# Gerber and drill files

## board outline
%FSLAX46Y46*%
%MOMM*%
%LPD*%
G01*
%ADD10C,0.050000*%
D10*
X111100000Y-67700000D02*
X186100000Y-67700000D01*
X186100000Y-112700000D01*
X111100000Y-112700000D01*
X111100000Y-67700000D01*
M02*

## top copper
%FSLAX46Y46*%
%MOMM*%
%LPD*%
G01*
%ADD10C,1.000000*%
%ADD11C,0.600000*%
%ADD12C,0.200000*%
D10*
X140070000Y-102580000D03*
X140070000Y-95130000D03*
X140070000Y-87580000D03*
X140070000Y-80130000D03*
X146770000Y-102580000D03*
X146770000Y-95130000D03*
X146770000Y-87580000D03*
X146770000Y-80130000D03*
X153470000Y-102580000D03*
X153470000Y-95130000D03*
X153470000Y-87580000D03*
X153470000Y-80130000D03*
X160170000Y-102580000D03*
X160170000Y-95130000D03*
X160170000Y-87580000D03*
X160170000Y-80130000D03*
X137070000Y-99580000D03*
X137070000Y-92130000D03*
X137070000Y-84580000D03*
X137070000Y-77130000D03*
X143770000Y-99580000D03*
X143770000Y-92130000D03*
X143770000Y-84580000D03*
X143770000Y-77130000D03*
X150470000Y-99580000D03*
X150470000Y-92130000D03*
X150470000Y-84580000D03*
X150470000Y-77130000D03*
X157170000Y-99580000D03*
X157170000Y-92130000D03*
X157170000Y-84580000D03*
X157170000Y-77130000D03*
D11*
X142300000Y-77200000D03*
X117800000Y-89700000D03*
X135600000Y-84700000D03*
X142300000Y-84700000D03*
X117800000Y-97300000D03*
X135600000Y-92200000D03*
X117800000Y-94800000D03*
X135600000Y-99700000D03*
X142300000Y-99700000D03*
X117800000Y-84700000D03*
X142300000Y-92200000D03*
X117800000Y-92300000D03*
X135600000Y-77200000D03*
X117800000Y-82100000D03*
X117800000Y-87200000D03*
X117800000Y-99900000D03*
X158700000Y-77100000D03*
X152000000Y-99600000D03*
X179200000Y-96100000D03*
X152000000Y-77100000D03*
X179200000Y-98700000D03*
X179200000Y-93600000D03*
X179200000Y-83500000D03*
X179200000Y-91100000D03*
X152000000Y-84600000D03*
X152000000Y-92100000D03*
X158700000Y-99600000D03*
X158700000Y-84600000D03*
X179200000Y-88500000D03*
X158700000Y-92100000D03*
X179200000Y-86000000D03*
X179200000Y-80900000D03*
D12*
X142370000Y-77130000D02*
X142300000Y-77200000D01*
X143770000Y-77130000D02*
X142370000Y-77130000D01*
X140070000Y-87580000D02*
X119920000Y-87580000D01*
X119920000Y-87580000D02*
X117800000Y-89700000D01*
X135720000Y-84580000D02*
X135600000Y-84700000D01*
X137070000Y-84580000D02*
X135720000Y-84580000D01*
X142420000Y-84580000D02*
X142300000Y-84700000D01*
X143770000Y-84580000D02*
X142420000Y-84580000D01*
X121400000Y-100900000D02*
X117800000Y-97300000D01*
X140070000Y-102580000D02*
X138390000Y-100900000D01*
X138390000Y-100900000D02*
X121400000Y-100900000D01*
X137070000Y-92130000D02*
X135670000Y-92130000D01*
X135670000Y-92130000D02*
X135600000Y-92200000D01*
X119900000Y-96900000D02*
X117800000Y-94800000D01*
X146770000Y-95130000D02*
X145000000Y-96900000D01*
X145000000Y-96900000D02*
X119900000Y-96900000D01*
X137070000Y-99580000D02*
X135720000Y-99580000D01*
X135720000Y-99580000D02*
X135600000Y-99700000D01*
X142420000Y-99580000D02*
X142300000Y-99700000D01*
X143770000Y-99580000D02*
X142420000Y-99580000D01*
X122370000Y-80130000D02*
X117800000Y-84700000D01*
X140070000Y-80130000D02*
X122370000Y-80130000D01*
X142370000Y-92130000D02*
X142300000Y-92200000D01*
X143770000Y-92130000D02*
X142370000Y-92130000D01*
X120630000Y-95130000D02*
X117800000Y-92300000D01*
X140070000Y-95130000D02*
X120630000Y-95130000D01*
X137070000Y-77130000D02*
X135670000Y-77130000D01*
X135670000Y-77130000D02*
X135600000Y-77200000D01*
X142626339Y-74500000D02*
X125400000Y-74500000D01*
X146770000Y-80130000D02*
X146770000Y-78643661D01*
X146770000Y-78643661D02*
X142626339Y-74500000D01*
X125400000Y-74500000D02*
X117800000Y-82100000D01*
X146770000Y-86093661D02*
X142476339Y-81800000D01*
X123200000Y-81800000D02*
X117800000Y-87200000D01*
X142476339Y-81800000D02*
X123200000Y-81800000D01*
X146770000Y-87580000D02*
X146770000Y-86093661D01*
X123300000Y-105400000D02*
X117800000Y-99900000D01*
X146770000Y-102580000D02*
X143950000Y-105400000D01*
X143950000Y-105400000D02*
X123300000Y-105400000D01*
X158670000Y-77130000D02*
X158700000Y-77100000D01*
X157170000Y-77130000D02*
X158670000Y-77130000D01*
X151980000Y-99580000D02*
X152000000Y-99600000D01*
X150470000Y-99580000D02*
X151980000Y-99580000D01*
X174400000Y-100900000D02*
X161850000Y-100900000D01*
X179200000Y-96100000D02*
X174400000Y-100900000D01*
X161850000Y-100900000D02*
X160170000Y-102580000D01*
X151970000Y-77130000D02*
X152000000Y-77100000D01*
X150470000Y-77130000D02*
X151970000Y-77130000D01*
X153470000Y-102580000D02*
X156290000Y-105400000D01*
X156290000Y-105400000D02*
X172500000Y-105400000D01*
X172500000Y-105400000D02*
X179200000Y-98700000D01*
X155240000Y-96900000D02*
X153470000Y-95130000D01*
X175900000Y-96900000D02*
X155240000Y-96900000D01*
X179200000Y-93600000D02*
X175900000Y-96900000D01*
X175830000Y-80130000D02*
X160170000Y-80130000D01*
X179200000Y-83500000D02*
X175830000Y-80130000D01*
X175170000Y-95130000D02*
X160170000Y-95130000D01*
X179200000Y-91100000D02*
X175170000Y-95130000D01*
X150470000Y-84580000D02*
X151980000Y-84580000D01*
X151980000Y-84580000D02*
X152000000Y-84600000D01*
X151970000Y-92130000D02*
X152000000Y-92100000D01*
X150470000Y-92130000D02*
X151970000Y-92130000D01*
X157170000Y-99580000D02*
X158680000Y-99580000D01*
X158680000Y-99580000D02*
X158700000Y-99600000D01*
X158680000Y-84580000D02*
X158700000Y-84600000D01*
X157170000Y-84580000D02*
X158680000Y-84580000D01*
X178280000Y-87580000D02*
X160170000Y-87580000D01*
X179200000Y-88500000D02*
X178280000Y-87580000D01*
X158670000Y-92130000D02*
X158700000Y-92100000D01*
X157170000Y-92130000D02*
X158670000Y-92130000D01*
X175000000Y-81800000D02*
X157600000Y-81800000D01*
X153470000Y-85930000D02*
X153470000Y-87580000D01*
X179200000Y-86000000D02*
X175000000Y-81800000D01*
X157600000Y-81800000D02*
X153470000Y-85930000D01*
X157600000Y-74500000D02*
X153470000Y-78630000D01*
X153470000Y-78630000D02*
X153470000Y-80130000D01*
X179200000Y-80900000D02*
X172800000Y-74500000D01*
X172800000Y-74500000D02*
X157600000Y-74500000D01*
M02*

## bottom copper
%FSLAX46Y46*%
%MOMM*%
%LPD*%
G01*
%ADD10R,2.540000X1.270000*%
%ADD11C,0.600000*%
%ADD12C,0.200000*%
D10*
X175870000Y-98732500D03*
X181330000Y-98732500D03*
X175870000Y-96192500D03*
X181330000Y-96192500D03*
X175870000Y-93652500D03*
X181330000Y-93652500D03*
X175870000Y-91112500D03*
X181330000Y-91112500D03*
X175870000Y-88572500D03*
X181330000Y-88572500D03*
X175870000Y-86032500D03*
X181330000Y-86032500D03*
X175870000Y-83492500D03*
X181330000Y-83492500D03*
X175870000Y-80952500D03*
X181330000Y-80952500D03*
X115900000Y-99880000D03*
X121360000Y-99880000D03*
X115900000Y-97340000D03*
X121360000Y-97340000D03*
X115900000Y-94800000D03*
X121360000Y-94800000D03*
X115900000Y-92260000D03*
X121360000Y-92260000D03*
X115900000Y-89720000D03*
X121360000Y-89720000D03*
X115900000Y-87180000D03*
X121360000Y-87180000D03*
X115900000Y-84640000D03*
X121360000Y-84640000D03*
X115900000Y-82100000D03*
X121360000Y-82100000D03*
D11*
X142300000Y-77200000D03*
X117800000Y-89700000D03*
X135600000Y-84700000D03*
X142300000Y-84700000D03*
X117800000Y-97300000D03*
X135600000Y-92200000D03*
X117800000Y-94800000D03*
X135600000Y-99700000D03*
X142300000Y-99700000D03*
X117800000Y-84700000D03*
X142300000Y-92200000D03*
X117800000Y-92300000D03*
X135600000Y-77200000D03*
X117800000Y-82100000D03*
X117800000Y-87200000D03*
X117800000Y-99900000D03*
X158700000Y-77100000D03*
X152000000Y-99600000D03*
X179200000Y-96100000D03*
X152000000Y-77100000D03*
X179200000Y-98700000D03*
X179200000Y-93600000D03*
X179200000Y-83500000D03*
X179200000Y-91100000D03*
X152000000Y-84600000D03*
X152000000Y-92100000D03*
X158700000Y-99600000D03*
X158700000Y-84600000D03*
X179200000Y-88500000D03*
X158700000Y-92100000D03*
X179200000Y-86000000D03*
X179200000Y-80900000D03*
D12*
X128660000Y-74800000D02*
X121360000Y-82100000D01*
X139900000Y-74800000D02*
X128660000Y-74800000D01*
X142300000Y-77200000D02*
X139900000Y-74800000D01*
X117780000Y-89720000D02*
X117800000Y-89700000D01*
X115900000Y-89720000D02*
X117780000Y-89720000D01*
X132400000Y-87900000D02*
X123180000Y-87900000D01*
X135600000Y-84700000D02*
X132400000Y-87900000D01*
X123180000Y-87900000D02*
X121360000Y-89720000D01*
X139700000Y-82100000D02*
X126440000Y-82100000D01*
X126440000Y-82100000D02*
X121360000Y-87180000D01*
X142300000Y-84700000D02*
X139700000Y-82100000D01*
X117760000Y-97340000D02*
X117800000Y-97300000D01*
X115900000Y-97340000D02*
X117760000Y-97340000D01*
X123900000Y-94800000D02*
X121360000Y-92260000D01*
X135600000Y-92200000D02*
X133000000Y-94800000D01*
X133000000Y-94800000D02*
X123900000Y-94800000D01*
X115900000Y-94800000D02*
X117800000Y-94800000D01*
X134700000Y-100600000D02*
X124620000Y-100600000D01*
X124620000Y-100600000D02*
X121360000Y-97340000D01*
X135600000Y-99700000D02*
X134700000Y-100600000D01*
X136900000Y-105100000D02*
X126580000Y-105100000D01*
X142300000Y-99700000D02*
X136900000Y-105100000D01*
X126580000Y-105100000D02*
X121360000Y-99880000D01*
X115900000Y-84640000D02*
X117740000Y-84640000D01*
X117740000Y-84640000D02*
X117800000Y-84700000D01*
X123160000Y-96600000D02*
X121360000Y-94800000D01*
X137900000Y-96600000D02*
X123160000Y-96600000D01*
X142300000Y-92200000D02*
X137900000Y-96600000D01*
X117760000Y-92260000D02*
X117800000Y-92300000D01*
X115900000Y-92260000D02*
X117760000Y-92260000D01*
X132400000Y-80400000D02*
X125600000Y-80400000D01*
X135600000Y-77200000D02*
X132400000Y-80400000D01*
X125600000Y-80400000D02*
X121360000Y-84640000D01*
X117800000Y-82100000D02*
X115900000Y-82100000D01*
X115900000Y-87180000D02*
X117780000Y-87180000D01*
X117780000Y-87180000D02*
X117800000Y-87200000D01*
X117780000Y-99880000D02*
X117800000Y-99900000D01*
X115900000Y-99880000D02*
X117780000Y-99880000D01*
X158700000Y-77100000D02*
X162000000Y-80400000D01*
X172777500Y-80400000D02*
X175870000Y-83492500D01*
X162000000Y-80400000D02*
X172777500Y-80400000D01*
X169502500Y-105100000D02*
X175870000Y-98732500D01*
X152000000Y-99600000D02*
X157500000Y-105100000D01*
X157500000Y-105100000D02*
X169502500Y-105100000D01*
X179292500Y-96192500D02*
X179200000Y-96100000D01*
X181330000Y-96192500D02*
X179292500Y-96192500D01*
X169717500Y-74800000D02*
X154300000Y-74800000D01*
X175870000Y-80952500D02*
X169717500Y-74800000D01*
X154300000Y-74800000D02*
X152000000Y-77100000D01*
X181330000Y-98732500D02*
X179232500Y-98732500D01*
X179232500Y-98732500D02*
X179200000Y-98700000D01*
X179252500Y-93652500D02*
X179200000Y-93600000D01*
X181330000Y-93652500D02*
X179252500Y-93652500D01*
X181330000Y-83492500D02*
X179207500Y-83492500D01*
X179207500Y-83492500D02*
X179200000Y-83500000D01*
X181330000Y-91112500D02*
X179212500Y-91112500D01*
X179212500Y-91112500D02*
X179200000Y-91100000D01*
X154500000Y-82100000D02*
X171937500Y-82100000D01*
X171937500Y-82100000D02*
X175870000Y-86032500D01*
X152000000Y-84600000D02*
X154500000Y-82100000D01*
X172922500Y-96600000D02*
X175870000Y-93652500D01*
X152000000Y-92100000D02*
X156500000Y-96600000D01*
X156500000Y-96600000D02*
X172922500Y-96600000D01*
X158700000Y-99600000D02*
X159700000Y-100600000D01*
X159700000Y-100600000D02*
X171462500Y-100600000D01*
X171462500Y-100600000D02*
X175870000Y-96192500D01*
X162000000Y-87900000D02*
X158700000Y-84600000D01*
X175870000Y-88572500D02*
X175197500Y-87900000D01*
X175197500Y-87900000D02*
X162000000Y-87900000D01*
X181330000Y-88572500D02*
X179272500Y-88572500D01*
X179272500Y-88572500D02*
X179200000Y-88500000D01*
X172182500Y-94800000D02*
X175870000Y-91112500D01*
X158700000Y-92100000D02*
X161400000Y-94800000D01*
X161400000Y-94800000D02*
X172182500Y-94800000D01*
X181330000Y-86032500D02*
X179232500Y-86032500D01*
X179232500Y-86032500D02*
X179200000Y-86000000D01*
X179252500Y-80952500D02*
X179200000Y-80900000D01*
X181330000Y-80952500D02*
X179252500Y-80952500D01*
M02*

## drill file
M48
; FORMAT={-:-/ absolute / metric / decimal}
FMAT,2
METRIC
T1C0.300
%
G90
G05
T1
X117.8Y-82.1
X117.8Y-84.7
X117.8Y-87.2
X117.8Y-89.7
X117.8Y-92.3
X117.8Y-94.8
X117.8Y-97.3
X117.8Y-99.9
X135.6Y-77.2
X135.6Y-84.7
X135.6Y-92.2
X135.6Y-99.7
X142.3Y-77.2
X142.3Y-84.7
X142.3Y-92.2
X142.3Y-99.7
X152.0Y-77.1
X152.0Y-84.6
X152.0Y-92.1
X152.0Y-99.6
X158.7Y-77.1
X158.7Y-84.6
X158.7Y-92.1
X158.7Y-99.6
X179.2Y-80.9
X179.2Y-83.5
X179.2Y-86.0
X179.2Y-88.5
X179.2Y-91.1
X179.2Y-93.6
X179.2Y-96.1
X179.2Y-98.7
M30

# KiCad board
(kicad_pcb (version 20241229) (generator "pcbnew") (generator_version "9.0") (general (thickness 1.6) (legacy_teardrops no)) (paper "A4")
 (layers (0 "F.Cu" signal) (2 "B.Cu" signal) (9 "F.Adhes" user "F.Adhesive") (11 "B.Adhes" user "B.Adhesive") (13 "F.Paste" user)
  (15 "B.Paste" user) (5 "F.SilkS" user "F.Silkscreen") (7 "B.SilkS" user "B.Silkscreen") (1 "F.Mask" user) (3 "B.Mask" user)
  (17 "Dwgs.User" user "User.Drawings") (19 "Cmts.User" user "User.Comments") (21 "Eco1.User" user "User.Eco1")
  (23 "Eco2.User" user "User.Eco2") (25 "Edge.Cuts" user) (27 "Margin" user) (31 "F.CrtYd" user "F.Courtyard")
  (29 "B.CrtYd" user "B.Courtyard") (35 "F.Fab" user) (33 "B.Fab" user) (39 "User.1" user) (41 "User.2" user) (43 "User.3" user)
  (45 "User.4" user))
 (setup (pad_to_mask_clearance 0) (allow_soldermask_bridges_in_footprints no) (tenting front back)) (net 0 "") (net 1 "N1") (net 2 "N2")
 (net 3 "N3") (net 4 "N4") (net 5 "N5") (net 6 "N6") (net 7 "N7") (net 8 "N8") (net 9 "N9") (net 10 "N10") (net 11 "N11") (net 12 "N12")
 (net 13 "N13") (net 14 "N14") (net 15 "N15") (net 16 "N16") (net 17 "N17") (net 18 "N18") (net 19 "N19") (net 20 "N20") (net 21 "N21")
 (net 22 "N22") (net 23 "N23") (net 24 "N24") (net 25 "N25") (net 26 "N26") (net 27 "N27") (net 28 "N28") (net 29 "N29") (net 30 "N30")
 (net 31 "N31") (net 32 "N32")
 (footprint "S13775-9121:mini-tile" (layer "F.Cu") (at 148.62 90.13)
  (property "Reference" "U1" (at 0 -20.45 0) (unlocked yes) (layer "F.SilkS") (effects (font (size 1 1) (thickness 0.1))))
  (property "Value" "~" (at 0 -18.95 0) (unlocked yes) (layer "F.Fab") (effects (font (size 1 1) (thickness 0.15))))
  (pad "AA1" smd circle (at -8.55 12.45) (size 1 1) (layers "F.Cu" "F.Mask" "F.Paste") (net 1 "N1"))
  (pad "AA2" smd circle (at -8.55 5) (size 1 1) (layers "F.Cu" "F.Mask" "F.Paste") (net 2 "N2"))
  (pad "AA3" smd circle (at -8.55 -2.55) (size 1 1) (layers "F.Cu" "F.Mask" "F.Paste") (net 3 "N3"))
  (pad "AA4" smd circle (at -8.55 -10) (size 1 1) (layers "F.Cu" "F.Mask" "F.Paste") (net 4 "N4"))
  (pad "AB1" smd circle (at -1.85 12.45) (size 1 1) (layers "F.Cu" "F.Mask" "F.Paste") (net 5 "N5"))
  (pad "AB2" smd circle (at -1.85 5) (size 1 1) (layers "F.Cu" "F.Mask" "F.Paste") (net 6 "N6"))
  (pad "AB3" smd circle (at -1.85 -2.55) (size 1 1) (layers "F.Cu" "F.Mask" "F.Paste") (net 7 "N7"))
  (pad "AB4" smd circle (at -1.85 -10) (size 1 1) (layers "F.Cu" "F.Mask" "F.Paste") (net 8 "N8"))
  (pad "AC1" smd circle (at 4.85 12.45) (size 1 1) (layers "F.Cu" "F.Mask" "F.Paste") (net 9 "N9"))
  (pad "AC2" smd circle (at 4.85 5) (size 1 1) (layers "F.Cu" "F.Mask" "F.Paste") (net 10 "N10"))
  (pad "AC3" smd circle (at 4.85 -2.55) (size 1 1) (layers "F.Cu" "F.Mask" "F.Paste") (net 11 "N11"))
  (pad "AC4" smd circle (at 4.85 -10) (size 1 1) (layers "F.Cu" "F.Mask" "F.Paste") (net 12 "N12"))
  (pad "AD1" smd circle (at 11.55 12.45) (size 1 1) (layers "F.Cu" "F.Mask" "F.Paste") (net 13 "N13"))
  (pad "AD2" smd circle (at 11.55 5) (size 1 1) (layers "F.Cu" "F.Mask" "F.Paste") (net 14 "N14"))
  (pad "AD3" smd circle (at 11.55 -2.55) (size 1 1) (layers "F.Cu" "F.Mask" "F.Paste") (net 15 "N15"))
  (pad "AD4" smd circle (at 11.55 -10) (size 1 1) (layers "F.Cu" "F.Mask" "F.Paste") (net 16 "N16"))
  (pad "KA1" smd circle (at -11.55 9.45) (size 1 1) (layers "F.Cu" "F.Mask" "F.Paste") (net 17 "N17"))
  (pad "KA2" smd circle (at -11.55 2) (size 1 1) (layers "F.Cu" "F.Mask" "F.Paste") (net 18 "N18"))
  (pad "KA3" smd circle (at -11.55 -5.55) (size 1 1) (layers "F.Cu" "F.Mask" "F.Paste") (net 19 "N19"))
  (pad "KA4" smd circle (at -11.55 -13) (size 1 1) (layers "F.Cu" "F.Mask" "F.Paste") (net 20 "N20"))
  (pad "KB1" smd circle (at -4.85 9.45) (size 1 1) (layers "F.Cu" "F.Mask" "F.Paste") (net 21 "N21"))
  (pad "KB2" smd circle (at -4.85 2) (size 1 1) (layers "F.Cu" "F.Mask" "F.Paste") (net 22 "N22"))
  (pad "KB3" smd circle (at -4.85 -5.55) (size 1 1) (layers "F.Cu" "F.Mask" "F.Paste") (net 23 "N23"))
  (pad "KB4" smd circle (at -4.85 -13) (size 1 1) (layers "F.Cu" "F.Mask" "F.Paste") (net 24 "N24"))
  (pad "KC1" smd circle (at 1.85 9.45) (size 1 1) (layers "F.Cu" "F.Mask" "F.Paste") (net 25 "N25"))
  (pad "KC2" smd circle (at 1.85 2) (size 1 1) (layers "F.Cu" "F.Mask" "F.Paste") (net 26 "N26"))
  (pad "KC3" smd circle (at 1.85 -5.55) (size 1 1) (layers "F.Cu" "F.Mask" "F.Paste") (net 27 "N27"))
  (pad "KC4" smd circle (at 1.85 -13) (size 1 1) (layers "F.Cu" "F.Mask" "F.Paste") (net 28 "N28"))
  (pad "KD1" smd circle (at 8.55 9.45) (size 1 1) (layers "F.Cu" "F.Mask" "F.Paste") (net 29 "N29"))
  (pad "KD2" smd circle (at 8.55 2) (size 1 1) (layers "F.Cu" "F.Mask" "F.Paste") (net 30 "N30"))
  (pad "KD3" smd circle (at 8.55 -5.55) (size 1 1) (layers "F.Cu" "F.Mask" "F.Paste") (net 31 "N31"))
  (pad "KD4" smd circle (at 8.55 -13) (size 1 1) (layers "F.Cu" "F.Mask" "F.Paste") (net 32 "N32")))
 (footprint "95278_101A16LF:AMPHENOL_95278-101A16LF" (layer "B.Cu") (at 178.6 89.8425 90)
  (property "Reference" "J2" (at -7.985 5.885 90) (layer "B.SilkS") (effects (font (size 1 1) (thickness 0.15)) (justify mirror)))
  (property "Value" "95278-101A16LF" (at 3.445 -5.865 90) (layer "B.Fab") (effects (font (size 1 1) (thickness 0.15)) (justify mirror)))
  (pad "01" smd rect (at -8.89 -2.73 90) (size 1.27 2.54) (layers "B.Cu" "B.Mask" "B.Paste") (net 25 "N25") (solder_mask_margin 0.102))
  (pad "02" smd rect (at -8.89 2.73 90) (size 1.27 2.54) (layers "B.Cu" "B.Mask" "B.Paste") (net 9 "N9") (solder_mask_margin 0.102))
  (pad "03" smd rect (at -6.35 -2.73 90) (size 1.27 2.54) (layers "B.Cu" "B.Mask" "B.Paste") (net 29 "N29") (solder_mask_margin 0.102))
  (pad "04" smd rect (at -6.35 2.73 90) (size 1.27 2.54) (layers "B.Cu" "B.Mask" "B.Paste") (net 13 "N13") (solder_mask_margin 0.102))
  (pad "05" smd rect (at -3.81 -2.73 90) (size 1.27 2.54) (layers "B.Cu" "B.Mask" "B.Paste") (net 26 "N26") (solder_mask_margin 0.102))
  (pad "06" smd rect (at -3.81 2.73 90) (size 1.27 2.54) (layers "B.Cu" "B.Mask" "B.Paste") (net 10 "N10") (solder_mask_margin 0.102))
  (pad "07" smd rect (at -1.27 -2.73 90) (size 1.27 2.54) (layers "B.Cu" "B.Mask" "B.Paste") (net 30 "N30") (solder_mask_margin 0.102))
  (pad "08" smd rect (at -1.27 2.73 90) (size 1.27 2.54) (layers "B.Cu" "B.Mask" "B.Paste") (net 14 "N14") (solder_mask_margin 0.102))
  (pad "09" smd rect (at 1.27 -2.73 90) (size 1.27 2.54) (layers "B.Cu" "B.Mask" "B.Paste") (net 31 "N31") (solder_mask_margin 0.102))
  (pad "10" smd rect (at 1.27 2.73 90) (size 1.27 2.54) (layers "B.Cu" "B.Mask" "B.Paste") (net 15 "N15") (solder_mask_margin 0.102))
  (pad "11" smd rect (at 3.81 -2.73 90) (size 1.27 2.54) (layers "B.Cu" "B.Mask" "B.Paste") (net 27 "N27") (solder_mask_margin 0.102))
  (pad "12" smd rect (at 3.81 2.73 90) (size 1.27 2.54) (layers "B.Cu" "B.Mask" "B.Paste") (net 11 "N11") (solder_mask_margin 0.102))
  (pad "13" smd rect (at 6.35 -2.73 90) (size 1.27 2.54) (layers "B.Cu" "B.Mask" "B.Paste") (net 32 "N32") (solder_mask_margin 0.102))
  (pad "14" smd rect (at 6.35 2.73 90) (size 1.27 2.54) (layers "B.Cu" "B.Mask" "B.Paste") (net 16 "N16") (solder_mask_margin 0.102))
  (pad "15" smd rect (at 8.89 -2.73 90) (size 1.27 2.54) (layers "B.Cu" "B.Mask" "B.Paste") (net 28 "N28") (solder_mask_margin 0.102))
  (pad "16" smd rect (at 8.89 2.73 90) (size 1.27 2.54) (layers "B.Cu" "B.Mask" "B.Paste") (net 12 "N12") (solder_mask_margin 0.102)))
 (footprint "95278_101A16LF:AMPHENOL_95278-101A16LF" (layer "B.Cu") (at 118.63 90.99 90)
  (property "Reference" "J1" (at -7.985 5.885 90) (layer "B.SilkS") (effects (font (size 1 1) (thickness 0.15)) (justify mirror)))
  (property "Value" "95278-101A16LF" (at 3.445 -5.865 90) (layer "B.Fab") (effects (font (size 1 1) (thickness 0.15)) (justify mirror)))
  (pad "01" smd rect (at -8.89 -2.73 90) (size 1.27 2.54) (layers "B.Cu" "B.Mask" "B.Paste") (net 5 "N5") (solder_mask_margin 0.102))
  (pad "02" smd rect (at -8.89 2.73 90) (size 1.27 2.54) (layers "B.Cu" "B.Mask" "B.Paste") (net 21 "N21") (solder_mask_margin 0.102))
  (pad "03" smd rect (at -6.35 -2.73 90) (size 1.27 2.54) (layers "B.Cu" "B.Mask" "B.Paste") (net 1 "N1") (solder_mask_margin 0.102))
  (pad "04" smd rect (at -6.35 2.73 90) (size 1.27 2.54) (layers "B.Cu" "B.Mask" "B.Paste") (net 17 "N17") (solder_mask_margin 0.102))
  (pad "05" smd rect (at -3.81 -2.73 90) (size 1.27 2.54) (layers "B.Cu" "B.Mask" "B.Paste") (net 6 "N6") (solder_mask_margin 0.102))
  (pad "06" smd rect (at -3.81 2.73 90) (size 1.27 2.54) (layers "B.Cu" "B.Mask" "B.Paste") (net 22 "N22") (solder_mask_margin 0.102))
  (pad "07" smd rect (at -1.27 -2.73 90) (size 1.27 2.54) (layers "B.Cu" "B.Mask" "B.Paste") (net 2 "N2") (solder_mask_margin 0.102))
  (pad "08" smd rect (at -1.27 2.73 90) (size 1.27 2.54) (layers "B.Cu" "B.Mask" "B.Paste") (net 18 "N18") (solder_mask_margin 0.102))
  (pad "09" smd rect (at 1.27 -2.73 90) (size 1.27 2.54) (layers "B.Cu" "B.Mask" "B.Paste") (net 3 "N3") (solder_mask_margin 0.102))
  (pad "10" smd rect (at 1.27 2.73 90) (size 1.27 2.54) (layers "B.Cu" "B.Mask" "B.Paste") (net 19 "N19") (solder_mask_margin 0.102))
  (pad "11" smd rect (at 3.81 -2.73 90) (size 1.27 2.54) (layers "B.Cu" "B.Mask" "B.Paste") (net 7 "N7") (solder_mask_margin 0.102))
  (pad "12" smd rect (at 3.81 2.73 90) (size 1.27 2.54) (layers "B.Cu" "B.Mask" "B.Paste") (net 23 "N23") (solder_mask_margin 0.102))
  (pad "13" smd rect (at 6.35 -2.73 90) (size 1.27 2.54) (layers "B.Cu" "B.Mask" "B.Paste") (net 4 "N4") (solder_mask_margin 0.102))
  (pad "14" smd rect (at 6.35 2.73 90) (size 1.27 2.54) (layers "B.Cu" "B.Mask" "B.Paste") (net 20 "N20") (solder_mask_margin 0.102))
  (pad "15" smd rect (at 8.89 -2.73 90) (size 1.27 2.54) (layers "B.Cu" "B.Mask" "B.Paste") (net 8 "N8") (solder_mask_margin 0.102))
  (pad "16" smd rect (at 8.89 2.73 90) (size 1.27 2.54) (layers "B.Cu" "B.Mask" "B.Paste") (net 24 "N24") (solder_mask_margin 0.102)))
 (gr_rect (start 111.1 67.7) (end 186.1 112.7) (stroke (width 0.05) (type solid)) (fill no) (layer "Edge.Cuts"))
 (segment (start 142.37 77.13) (end 142.3 77.2) (width 0.2) (layer "F.Cu") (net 24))
 (segment (start 143.77 77.13) (end 142.37 77.13) (width 0.2) (layer "F.Cu") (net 24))
 (via (at 142.3 77.2) (size 0.6) (drill 0.3) (layers "F.Cu" "B.Cu") (free yes) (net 24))
 (segment (start 128.66 74.8) (end 121.36 82.1) (width 0.2) (layer "B.Cu") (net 24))
 (segment (start 139.9 74.8) (end 128.66 74.8) (width 0.2) (layer "B.Cu") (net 24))
 (segment (start 142.3 77.2) (end 139.9 74.8) (width 0.2) (layer "B.Cu") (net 24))
 (segment (start 140.07 87.58) (end 119.92 87.58) (width 0.2) (layer "F.Cu") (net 3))
 (segment (start 119.92 87.58) (end 117.8 89.7) (width 0.2) (layer "F.Cu") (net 3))
 (via (at 117.8 89.7) (size 0.6) (drill 0.3) (layers "F.Cu" "B.Cu") (free yes) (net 3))
 (segment (start 117.78 89.72) (end 117.8 89.7) (width 0.2) (layer "B.Cu") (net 3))
 (segment (start 115.9 89.72) (end 117.78 89.72) (width 0.2) (layer "B.Cu") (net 3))
 (segment (start 135.72 84.58) (end 135.6 84.7) (width 0.2) (layer "F.Cu") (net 19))
 (segment (start 137.07 84.58) (end 135.72 84.58) (width 0.2) (layer "F.Cu") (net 19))
 (via (at 135.6 84.7) (size 0.6) (drill 0.3) (layers "F.Cu" "B.Cu") (free yes) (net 19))
 (segment (start 132.4 87.9) (end 123.18 87.9) (width 0.2) (layer "B.Cu") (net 19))
 (segment (start 135.6 84.7) (end 132.4 87.9) (width 0.2) (layer "B.Cu") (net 19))
 (segment (start 123.18 87.9) (end 121.36 89.72) (width 0.2) (layer "B.Cu") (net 19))
 (segment (start 142.42 84.58) (end 142.3 84.7) (width 0.2) (layer "F.Cu") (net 23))
 (segment (start 143.77 84.58) (end 142.42 84.58) (width 0.2) (layer "F.Cu") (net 23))
 (via (at 142.3 84.7) (size 0.6) (drill 0.3) (layers "F.Cu" "B.Cu") (free yes) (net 23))
 (segment (start 139.7 82.1) (end 126.44 82.1) (width 0.2) (layer "B.Cu") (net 23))
 (segment (start 126.44 82.1) (end 121.36 87.18) (width 0.2) (layer "B.Cu") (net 23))
 (segment (start 142.3 84.7) (end 139.7 82.1) (width 0.2) (layer "B.Cu") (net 23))
 (segment (start 121.4 100.9) (end 117.8 97.3) (width 0.2) (layer "F.Cu") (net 1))
 (segment (start 140.07 102.58) (end 138.39 100.9) (width 0.2) (layer "F.Cu") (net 1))
 (segment (start 138.39 100.9) (end 121.4 100.9) (width 0.2) (layer "F.Cu") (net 1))
 (via (at 117.8 97.3) (size 0.6) (drill 0.3) (layers "F.Cu" "B.Cu") (free yes) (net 1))
 (segment (start 117.76 97.34) (end 117.8 97.3) (width 0.2) (layer "B.Cu") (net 1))
 (segment (start 115.9 97.34) (end 117.76 97.34) (width 0.2) (layer "B.Cu") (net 1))
 (segment (start 137.07 92.13) (end 135.67 92.13) (width 0.2) (layer "F.Cu") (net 18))
 (segment (start 135.67 92.13) (end 135.6 92.2) (width 0.2) (layer "F.Cu") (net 18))
 (via (at 135.6 92.2) (size 0.6) (drill 0.3) (layers "F.Cu" "B.Cu") (free yes) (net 18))
 (segment (start 123.9 94.8) (end 121.36 92.26) (width 0.2) (layer "B.Cu") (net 18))
 (segment (start 135.6 92.2) (end 133 94.8) (width 0.2) (layer "B.Cu") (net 18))
 (segment (start 133 94.8) (end 123.9 94.8) (width 0.2) (layer "B.Cu") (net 18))
 (segment (start 119.9 96.9) (end 117.8 94.8) (width 0.2) (layer "F.Cu") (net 6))
 (segment (start 146.77 95.13) (end 145 96.9) (width 0.2) (layer "F.Cu") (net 6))
 (segment (start 145 96.9) (end 119.9 96.9) (width 0.2) (layer "F.Cu") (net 6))
 (via (at 117.8 94.8) (size 0.6) (drill 0.3) (layers "F.Cu" "B.Cu") (free yes) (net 6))
 (segment (start 115.9 94.8) (end 117.8 94.8) (width 0.2) (layer "B.Cu") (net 6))
 (segment (start 137.07 99.58) (end 135.72 99.58) (width 0.2) (layer "F.Cu") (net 17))
 (segment (start 135.72 99.58) (end 135.6 99.7) (width 0.2) (layer "F.Cu") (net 17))
 (via (at 135.6 99.7) (size 0.6) (drill 0.3) (layers "F.Cu" "B.Cu") (free yes) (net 17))
 (segment (start 134.7 100.6) (end 124.62 100.6) (width 0.2) (layer "B.Cu") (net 17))
 (segment (start 124.62 100.6) (end 121.36 97.34) (width 0.2) (layer "B.Cu") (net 17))
 (segment (start 135.6 99.7) (end 134.7 100.6) (width 0.2) (layer "B.Cu") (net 17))
 (segment (start 142.42 99.58) (end 142.3 99.7) (width 0.2) (layer "F.Cu") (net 21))
 (segment (start 143.77 99.58) (end 142.42 99.58) (width 0.2) (layer "F.Cu") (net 21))
 (via (at 142.3 99.7) (size 0.6) (drill 0.3) (layers "F.Cu" "B.Cu") (free yes) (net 21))
 (segment (start 136.9 105.1) (end 126.58 105.1) (width 0.2) (layer "B.Cu") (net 21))
 (segment (start 142.3 99.7) (end 136.9 105.1) (width 0.2) (layer "B.Cu") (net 21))
 (segment (start 126.58 105.1) (end 121.36 99.88) (width 0.2) (layer "B.Cu") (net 21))
 (segment (start 122.37 80.13) (end 117.8 84.7) (width 0.2) (layer "F.Cu") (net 4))
 (segment (start 140.07 80.13) (end 122.37 80.13) (width 0.2) (layer "F.Cu") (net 4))
 (via (at 117.8 84.7) (size 0.6) (drill 0.3) (layers "F.Cu" "B.Cu") (free yes) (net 4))
 (segment (start 115.9 84.64) (end 117.74 84.64) (width 0.2) (layer "B.Cu") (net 4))
 (segment (start 117.74 84.64) (end 117.8 84.7) (width 0.2) (layer "B.Cu") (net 4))
 (segment (start 142.37 92.13) (end 142.3 92.2) (width 0.2) (layer "F.Cu") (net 22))
 (segment (start 143.77 92.13) (end 142.37 92.13) (width 0.2) (layer "F.Cu") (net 22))
 (via (at 142.3 92.2) (size 0.6) (drill 0.3) (layers "F.Cu" "B.Cu") (free yes) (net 22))
 (segment (start 123.16 96.6) (end 121.36 94.8) (width 0.2) (layer "B.Cu") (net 22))
 (segment (start 137.9 96.6) (end 123.16 96.6) (width 0.2) (layer "B.Cu") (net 22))
 (segment (start 142.3 92.2) (end 137.9 96.6) (width 0.2) (layer "B.Cu") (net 22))
 (segment (start 120.63 95.13) (end 117.8 92.3) (width 0.2) (layer "F.Cu") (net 2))
 (segment (start 140.07 95.13) (end 120.63 95.13) (width 0.2) (layer "F.Cu") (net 2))
 (via (at 117.8 92.3) (size 0.6) (drill 0.3) (layers "F.Cu" "B.Cu") (free yes) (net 2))
 (segment (start 117.76 92.26) (end 117.8 92.3) (width 0.2) (layer "B.Cu") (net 2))
 (segment (start 115.9 92.26) (end 117.76 92.26) (width 0.2) (layer "B.Cu") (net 2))
 (segment (start 137.07 77.13) (end 135.67 77.13) (width 0.2) (layer "F.Cu") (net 20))
 (segment (start 135.67 77.13) (end 135.6 77.2) (width 0.2) (layer "F.Cu") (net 20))
 (via (at 135.6 77.2) (size 0.6) (drill 0.3) (layers "F.Cu" "B.Cu") (free yes) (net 20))
 (segment (start 132.4 80.4) (end 125.6 80.4) (width 0.2) (layer "B.Cu") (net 20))
 (segment (start 135.6 77.2) (end 132.4 80.4) (width 0.2) (layer "B.Cu") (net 20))
 (segment (start 125.6 80.4) (end 121.36 84.64) (width 0.2) (layer "B.Cu") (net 20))
 (segment (start 142.626339 74.5) (end 125.4 74.5) (width 0.2) (layer "F.Cu") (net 8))
 (segment (start 146.77 80.13) (end 146.77 78.643661) (width 0.2) (layer "F.Cu") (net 8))
 (segment (start 146.77 78.643661) (end 142.626339 74.5) (width 0.2) (layer "F.Cu") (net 8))
 (segment (start 125.4 74.5) (end 117.8 82.1) (width 0.2) (layer "F.Cu") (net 8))
 (via (at 117.8 82.1) (size 0.6) (drill 0.3) (layers "F.Cu" "B.Cu") (free yes) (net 8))
 (segment (start 117.8 82.1) (end 115.9 82.1) (width 0.2) (layer "B.Cu") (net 8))
 (segment (start 146.77 86.093661) (end 142.476339 81.8) (width 0.2) (layer "F.Cu") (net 7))
 (segment (start 123.2 81.8) (end 117.8 87.2) (width 0.2) (layer "F.Cu") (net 7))
 (segment (start 142.476339 81.8) (end 123.2 81.8) (width 0.2) (layer "F.Cu") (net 7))
 (segment (start 146.77 87.58) (end 146.77 86.093661) (width 0.2) (layer "F.Cu") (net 7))
 (via (at 117.8 87.2) (size 0.6) (drill 0.3) (layers "F.Cu" "B.Cu") (free yes) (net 7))
 (segment (start 115.9 87.18) (end 117.78 87.18) (width 0.2) (layer "B.Cu") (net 7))
 (segment (start 117.78 87.18) (end 117.8 87.2) (width 0.2) (layer "B.Cu") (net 7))
 (segment (start 123.3 105.4) (end 117.8 99.9) (width 0.2) (layer "F.Cu") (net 5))
 (segment (start 146.77 102.58) (end 143.95 105.4) (width 0.2) (layer "F.Cu") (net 5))
 (segment (start 143.95 105.4) (end 123.3 105.4) (width 0.2) (layer "F.Cu") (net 5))
 (via (at 117.8 99.9) (size 0.6) (drill 0.3) (layers "F.Cu" "B.Cu") (free yes) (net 5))
 (segment (start 117.78 99.88) (end 117.8 99.9) (width 0.2) (layer "B.Cu") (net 5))
 (segment (start 115.9 99.88) (end 117.78 99.88) (width 0.2) (layer "B.Cu") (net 5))
 (segment (start 158.67 77.13) (end 158.7 77.1) (width 0.2) (layer "F.Cu") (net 32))
 (segment (start 157.17 77.13) (end 158.67 77.13) (width 0.2) (layer "F.Cu") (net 32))
 (via (at 158.7 77.1) (size 0.6) (drill 0.3) (layers "F.Cu" "B.Cu") (free yes) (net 32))
 (segment (start 158.7 77.1) (end 162 80.4) (width 0.2) (layer "B.Cu") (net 32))
 (segment (start 172.7775 80.4) (end 175.87 83.4925) (width 0.2) (layer "B.Cu") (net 32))
 (segment (start 162 80.4) (end 172.7775 80.4) (width 0.2) (layer "B.Cu") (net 32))
 (segment (start 151.98 99.58) (end 152 99.6) (width 0.2) (layer "F.Cu") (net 25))
 (segment (start 150.47 99.58) (end 151.98 99.58) (width 0.2) (layer "F.Cu") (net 25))
 (via (at 152 99.6) (size 0.6) (drill 0.3) (layers "F.Cu" "B.Cu") (free yes) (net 25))
 (segment (start 169.5025 105.1) (end 175.87 98.7325) (width 0.2) (layer "B.Cu") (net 25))
 (segment (start 152 99.6) (end 157.5 105.1) (width 0.2) (layer "B.Cu") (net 25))
 (segment (start 157.5 105.1) (end 169.5025 105.1) (width 0.2) (layer "B.Cu") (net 25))
 (segment (start 174.4 100.9) (end 161.85 100.9) (width 0.2) (layer "F.Cu") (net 13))
 (segment (start 179.2 96.1) (end 174.4 100.9) (width 0.2) (layer "F.Cu") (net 13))
 (segment (start 161.85 100.9) (end 160.17 102.58) (width 0.2) (layer "F.Cu") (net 13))
 (via (at 179.2 96.1) (size 0.6) (drill 0.3) (layers "F.Cu" "B.Cu") (free yes) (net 13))
 (segment (start 179.2925 96.1925) (end 179.2 96.1) (width 0.2) (layer "B.Cu") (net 13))
 (segment (start 181.33 96.1925) (end 179.2925 96.1925) (width 0.2) (layer "B.Cu") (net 13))
 (segment (start 151.97 77.13) (end 152 77.1) (width 0.2) (layer "F.Cu") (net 28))
 (segment (start 150.47 77.13) (end 151.97 77.13) (width 0.2) (layer "F.Cu") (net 28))
 (via (at 152 77.1) (size 0.6) (drill 0.3) (layers "F.Cu" "B.Cu") (free yes) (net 28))
 (segment (start 169.7175 74.8) (end 154.3 74.8) (width 0.2) (layer "B.Cu") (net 28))
 (segment (start 175.87 80.9525) (end 169.7175 74.8) (width 0.2) (layer "B.Cu") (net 28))
 (segment (start 154.3 74.8) (end 152 77.1) (width 0.2) (layer "B.Cu") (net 28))
 (segment (start 153.47 102.58) (end 156.29 105.4) (width 0.2) (layer "F.Cu") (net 9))
 (segment (start 156.29 105.4) (end 172.5 105.4) (width 0.2) (layer "F.Cu") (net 9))
 (segment (start 172.5 105.4) (end 179.2 98.7) (width 0.2) (layer "F.Cu") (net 9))
 (via (at 179.2 98.7) (size 0.6) (drill 0.3) (layers "F.Cu" "B.Cu") (free yes) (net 9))
 (segment (start 181.33 98.7325) (end 179.2325 98.7325) (width 0.2) (layer "B.Cu") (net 9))
 (segment (start 179.2325 98.7325) (end 179.2 98.7) (width 0.2) (layer "B.Cu") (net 9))
 (segment (start 155.24 96.9) (end 153.47 95.13) (width 0.2) (layer "F.Cu") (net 10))
 (segment (start 175.9 96.9) (end 155.24 96.9) (width 0.2) (layer "F.Cu") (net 10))
 (segment (start 179.2 93.6) (end 175.9 96.9) (width 0.2) (layer "F.Cu") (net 10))
 (via (at 179.2 93.6) (size 0.6) (drill 0.3) (layers "F.Cu" "B.Cu") (free yes) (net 10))
 (segment (start 179.2525 93.6525) (end 179.2 93.6) (width 0.2) (layer "B.Cu") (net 10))
 (segment (start 181.33 93.6525) (end 179.2525 93.6525) (width 0.2) (layer "B.Cu") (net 10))
 (segment (start 175.83 80.13) (end 160.17 80.13) (width 0.2) (layer "F.Cu") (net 16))
 (segment (start 179.2 83.5) (end 175.83 80.13) (width 0.2) (layer "F.Cu") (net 16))
 (via (at 179.2 83.5) (size 0.6) (drill 0.3) (layers "F.Cu" "B.Cu") (free yes) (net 16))
 (segment (start 181.33 83.4925) (end 179.2075 83.4925) (width 0.2) (layer "B.Cu") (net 16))
 (segment (start 179.2075 83.4925) (end 179.2 83.5) (width 0.2) (layer "B.Cu") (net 16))
 (segment (start 175.17 95.13) (end 160.17 95.13) (width 0.2) (layer "F.Cu") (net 14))
 (segment (start 179.2 91.1) (end 175.17 95.13) (width 0.2) (layer "F.Cu") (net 14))
 (via (at 179.2 91.1) (size 0.6) (drill 0.3) (layers "F.Cu" "B.Cu") (free yes) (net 14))
 (segment (start 181.33 91.1125) (end 179.2125 91.1125) (width 0.2) (layer "B.Cu") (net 14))
 (segment (start 179.2125 91.1125) (end 179.2 91.1) (width 0.2) (layer "B.Cu") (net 14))
 (segment (start 150.47 84.58) (end 151.98 84.58) (width 0.2) (layer "F.Cu") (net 27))
 (segment (start 151.98 84.58) (end 152 84.6) (width 0.2) (layer "F.Cu") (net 27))
 (via (at 152 84.6) (size 0.6) (drill 0.3) (layers "F.Cu" "B.Cu") (free yes) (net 27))
 (segment (start 154.5 82.1) (end 171.9375 82.1) (width 0.2) (layer "B.Cu") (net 27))
 (segment (start 171.9375 82.1) (end 175.87 86.0325) (width 0.2) (layer "B.Cu") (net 27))
 (segment (start 152 84.6) (end 154.5 82.1) (width 0.2) (layer "B.Cu") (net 27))
 (segment (start 151.97 92.13) (end 152 92.1) (width 0.2) (layer "F.Cu") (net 26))
 (segment (start 150.47 92.13) (end 151.97 92.13) (width 0.2) (layer "F.Cu") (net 26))
 (via (at 152 92.1) (size 0.6) (drill 0.3) (layers "F.Cu" "B.Cu") (free yes) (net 26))
 (segment (start 172.9225 96.6) (end 175.87 93.6525) (width 0.2) (layer "B.Cu") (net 26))
 (segment (start 152 92.1) (end 156.5 96.6) (width 0.2) (layer "B.Cu") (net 26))
 (segment (start 156.5 96.6) (end 172.9225 96.6) (width 0.2) (layer "B.Cu") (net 26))
 (segment (start 157.17 99.58) (end 158.68 99.58) (width 0.2) (layer "F.Cu") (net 29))
 (segment (start 158.68 99.58) (end 158.7 99.6) (width 0.2) (layer "F.Cu") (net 29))
 (via (at 158.7 99.6) (size 0.6) (drill 0.3) (layers "F.Cu" "B.Cu") (free yes) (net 29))
 (segment (start 158.7 99.6) (end 159.7 100.6) (width 0.2) (layer "B.Cu") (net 29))
 (segment (start 159.7 100.6) (end 171.4625 100.6) (width 0.2) (layer "B.Cu") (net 29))
 (segment (start 171.4625 100.6) (end 175.87 96.1925) (width 0.2) (layer "B.Cu") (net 29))
 (segment (start 158.68 84.58) (end 158.7 84.6) (width 0.2) (layer "F.Cu") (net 31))
 (segment (start 157.17 84.58) (end 158.68 84.58) (width 0.2) (layer "F.Cu") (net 31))
 (via (at 158.7 84.6) (size 0.6) (drill 0.3) (layers "F.Cu" "B.Cu") (free yes) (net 31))
 (segment (start 162 87.9) (end 158.7 84.6) (width 0.2) (layer "B.Cu") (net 31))
 (segment (start 175.87 88.5725) (end 175.1975 87.9) (width 0.2) (layer "B.Cu") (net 31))
 (segment (start 175.1975 87.9) (end 162 87.9) (width 0.2) (layer "B.Cu") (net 31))
 (segment (start 178.28 87.58) (end 160.17 87.58) (width 0.2) (layer "F.Cu") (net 15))
 (segment (start 179.2 88.5) (end 178.28 87.58) (width 0.2) (layer "F.Cu") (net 15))
 (via (at 179.2 88.5) (size 0.6) (drill 0.3) (layers "F.Cu" "B.Cu") (free yes) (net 15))
 (segment (start 181.33 88.5725) (end 179.2725 88.5725) (width 0.2) (layer "B.Cu") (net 15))
 (segment (start 179.2725 88.5725) (end 179.2 88.5) (width 0.2) (layer "B.Cu") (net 15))
 (segment (start 158.67 92.13) (end 158.7 92.1) (width 0.2) (layer "F.Cu") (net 30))
 (segment (start 157.17 92.13) (end 158.67 92.13) (width 0.2) (layer "F.Cu") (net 30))
 (via (at 158.7 92.1) (size 0.6) (drill 0.3) (layers "F.Cu" "B.Cu") (free yes) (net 30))
 (segment (start 172.1825 94.8) (end 175.87 91.1125) (width 0.2) (layer "B.Cu") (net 30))
 (segment (start 158.7 92.1) (end 161.4 94.8) (width 0.2) (layer "B.Cu") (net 30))
 (segment (start 161.4 94.8) (end 172.1825 94.8) (width 0.2) (layer "B.Cu") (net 30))
 (segment (start 175 81.8) (end 157.6 81.8) (width 0.2) (layer "F.Cu") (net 11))
 (segment (start 153.47 85.93) (end 153.47 87.58) (width 0.2) (layer "F.Cu") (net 11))
 (segment (start 179.2 86) (end 175 81.8) (width 0.2) (layer "F.Cu") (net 11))
 (segment (start 157.6 81.8) (end 153.47 85.93) (width 0.2) (layer "F.Cu") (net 11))
 (via (at 179.2 86) (size 0.6) (drill 0.3) (layers "F.Cu" "B.Cu") (free yes) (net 11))
 (segment (start 181.33 86.0325) (end 179.2325 86.0325) (width 0.2) (layer "B.Cu") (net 11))
 (segment (start 179.2325 86.0325) (end 179.2 86) (width 0.2) (layer "B.Cu") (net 11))
 (segment (start 157.6 74.5) (end 153.47 78.63) (width 0.2) (layer "F.Cu") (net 12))
 (segment (start 153.47 78.63) (end 153.47 80.13) (width 0.2) (layer "F.Cu") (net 12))
 (segment (start 179.2 80.9) (end 172.8 74.5) (width 0.2) (layer "F.Cu") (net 12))
 (segment (start 172.8 74.5) (end 157.6 74.5) (width 0.2) (layer "F.Cu") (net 12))
 (via (at 179.2 80.9) (size 0.6) (drill 0.3) (layers "F.Cu" "B.Cu") (free yes) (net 12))
 (segment (start 179.2525 80.9525) (end 179.2 80.9) (width 0.2) (layer "B.Cu") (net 12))
 (segment (start 181.33 80.9525) (end 179.2525 80.9525) (width 0.2) (layer "B.Cu") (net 12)))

